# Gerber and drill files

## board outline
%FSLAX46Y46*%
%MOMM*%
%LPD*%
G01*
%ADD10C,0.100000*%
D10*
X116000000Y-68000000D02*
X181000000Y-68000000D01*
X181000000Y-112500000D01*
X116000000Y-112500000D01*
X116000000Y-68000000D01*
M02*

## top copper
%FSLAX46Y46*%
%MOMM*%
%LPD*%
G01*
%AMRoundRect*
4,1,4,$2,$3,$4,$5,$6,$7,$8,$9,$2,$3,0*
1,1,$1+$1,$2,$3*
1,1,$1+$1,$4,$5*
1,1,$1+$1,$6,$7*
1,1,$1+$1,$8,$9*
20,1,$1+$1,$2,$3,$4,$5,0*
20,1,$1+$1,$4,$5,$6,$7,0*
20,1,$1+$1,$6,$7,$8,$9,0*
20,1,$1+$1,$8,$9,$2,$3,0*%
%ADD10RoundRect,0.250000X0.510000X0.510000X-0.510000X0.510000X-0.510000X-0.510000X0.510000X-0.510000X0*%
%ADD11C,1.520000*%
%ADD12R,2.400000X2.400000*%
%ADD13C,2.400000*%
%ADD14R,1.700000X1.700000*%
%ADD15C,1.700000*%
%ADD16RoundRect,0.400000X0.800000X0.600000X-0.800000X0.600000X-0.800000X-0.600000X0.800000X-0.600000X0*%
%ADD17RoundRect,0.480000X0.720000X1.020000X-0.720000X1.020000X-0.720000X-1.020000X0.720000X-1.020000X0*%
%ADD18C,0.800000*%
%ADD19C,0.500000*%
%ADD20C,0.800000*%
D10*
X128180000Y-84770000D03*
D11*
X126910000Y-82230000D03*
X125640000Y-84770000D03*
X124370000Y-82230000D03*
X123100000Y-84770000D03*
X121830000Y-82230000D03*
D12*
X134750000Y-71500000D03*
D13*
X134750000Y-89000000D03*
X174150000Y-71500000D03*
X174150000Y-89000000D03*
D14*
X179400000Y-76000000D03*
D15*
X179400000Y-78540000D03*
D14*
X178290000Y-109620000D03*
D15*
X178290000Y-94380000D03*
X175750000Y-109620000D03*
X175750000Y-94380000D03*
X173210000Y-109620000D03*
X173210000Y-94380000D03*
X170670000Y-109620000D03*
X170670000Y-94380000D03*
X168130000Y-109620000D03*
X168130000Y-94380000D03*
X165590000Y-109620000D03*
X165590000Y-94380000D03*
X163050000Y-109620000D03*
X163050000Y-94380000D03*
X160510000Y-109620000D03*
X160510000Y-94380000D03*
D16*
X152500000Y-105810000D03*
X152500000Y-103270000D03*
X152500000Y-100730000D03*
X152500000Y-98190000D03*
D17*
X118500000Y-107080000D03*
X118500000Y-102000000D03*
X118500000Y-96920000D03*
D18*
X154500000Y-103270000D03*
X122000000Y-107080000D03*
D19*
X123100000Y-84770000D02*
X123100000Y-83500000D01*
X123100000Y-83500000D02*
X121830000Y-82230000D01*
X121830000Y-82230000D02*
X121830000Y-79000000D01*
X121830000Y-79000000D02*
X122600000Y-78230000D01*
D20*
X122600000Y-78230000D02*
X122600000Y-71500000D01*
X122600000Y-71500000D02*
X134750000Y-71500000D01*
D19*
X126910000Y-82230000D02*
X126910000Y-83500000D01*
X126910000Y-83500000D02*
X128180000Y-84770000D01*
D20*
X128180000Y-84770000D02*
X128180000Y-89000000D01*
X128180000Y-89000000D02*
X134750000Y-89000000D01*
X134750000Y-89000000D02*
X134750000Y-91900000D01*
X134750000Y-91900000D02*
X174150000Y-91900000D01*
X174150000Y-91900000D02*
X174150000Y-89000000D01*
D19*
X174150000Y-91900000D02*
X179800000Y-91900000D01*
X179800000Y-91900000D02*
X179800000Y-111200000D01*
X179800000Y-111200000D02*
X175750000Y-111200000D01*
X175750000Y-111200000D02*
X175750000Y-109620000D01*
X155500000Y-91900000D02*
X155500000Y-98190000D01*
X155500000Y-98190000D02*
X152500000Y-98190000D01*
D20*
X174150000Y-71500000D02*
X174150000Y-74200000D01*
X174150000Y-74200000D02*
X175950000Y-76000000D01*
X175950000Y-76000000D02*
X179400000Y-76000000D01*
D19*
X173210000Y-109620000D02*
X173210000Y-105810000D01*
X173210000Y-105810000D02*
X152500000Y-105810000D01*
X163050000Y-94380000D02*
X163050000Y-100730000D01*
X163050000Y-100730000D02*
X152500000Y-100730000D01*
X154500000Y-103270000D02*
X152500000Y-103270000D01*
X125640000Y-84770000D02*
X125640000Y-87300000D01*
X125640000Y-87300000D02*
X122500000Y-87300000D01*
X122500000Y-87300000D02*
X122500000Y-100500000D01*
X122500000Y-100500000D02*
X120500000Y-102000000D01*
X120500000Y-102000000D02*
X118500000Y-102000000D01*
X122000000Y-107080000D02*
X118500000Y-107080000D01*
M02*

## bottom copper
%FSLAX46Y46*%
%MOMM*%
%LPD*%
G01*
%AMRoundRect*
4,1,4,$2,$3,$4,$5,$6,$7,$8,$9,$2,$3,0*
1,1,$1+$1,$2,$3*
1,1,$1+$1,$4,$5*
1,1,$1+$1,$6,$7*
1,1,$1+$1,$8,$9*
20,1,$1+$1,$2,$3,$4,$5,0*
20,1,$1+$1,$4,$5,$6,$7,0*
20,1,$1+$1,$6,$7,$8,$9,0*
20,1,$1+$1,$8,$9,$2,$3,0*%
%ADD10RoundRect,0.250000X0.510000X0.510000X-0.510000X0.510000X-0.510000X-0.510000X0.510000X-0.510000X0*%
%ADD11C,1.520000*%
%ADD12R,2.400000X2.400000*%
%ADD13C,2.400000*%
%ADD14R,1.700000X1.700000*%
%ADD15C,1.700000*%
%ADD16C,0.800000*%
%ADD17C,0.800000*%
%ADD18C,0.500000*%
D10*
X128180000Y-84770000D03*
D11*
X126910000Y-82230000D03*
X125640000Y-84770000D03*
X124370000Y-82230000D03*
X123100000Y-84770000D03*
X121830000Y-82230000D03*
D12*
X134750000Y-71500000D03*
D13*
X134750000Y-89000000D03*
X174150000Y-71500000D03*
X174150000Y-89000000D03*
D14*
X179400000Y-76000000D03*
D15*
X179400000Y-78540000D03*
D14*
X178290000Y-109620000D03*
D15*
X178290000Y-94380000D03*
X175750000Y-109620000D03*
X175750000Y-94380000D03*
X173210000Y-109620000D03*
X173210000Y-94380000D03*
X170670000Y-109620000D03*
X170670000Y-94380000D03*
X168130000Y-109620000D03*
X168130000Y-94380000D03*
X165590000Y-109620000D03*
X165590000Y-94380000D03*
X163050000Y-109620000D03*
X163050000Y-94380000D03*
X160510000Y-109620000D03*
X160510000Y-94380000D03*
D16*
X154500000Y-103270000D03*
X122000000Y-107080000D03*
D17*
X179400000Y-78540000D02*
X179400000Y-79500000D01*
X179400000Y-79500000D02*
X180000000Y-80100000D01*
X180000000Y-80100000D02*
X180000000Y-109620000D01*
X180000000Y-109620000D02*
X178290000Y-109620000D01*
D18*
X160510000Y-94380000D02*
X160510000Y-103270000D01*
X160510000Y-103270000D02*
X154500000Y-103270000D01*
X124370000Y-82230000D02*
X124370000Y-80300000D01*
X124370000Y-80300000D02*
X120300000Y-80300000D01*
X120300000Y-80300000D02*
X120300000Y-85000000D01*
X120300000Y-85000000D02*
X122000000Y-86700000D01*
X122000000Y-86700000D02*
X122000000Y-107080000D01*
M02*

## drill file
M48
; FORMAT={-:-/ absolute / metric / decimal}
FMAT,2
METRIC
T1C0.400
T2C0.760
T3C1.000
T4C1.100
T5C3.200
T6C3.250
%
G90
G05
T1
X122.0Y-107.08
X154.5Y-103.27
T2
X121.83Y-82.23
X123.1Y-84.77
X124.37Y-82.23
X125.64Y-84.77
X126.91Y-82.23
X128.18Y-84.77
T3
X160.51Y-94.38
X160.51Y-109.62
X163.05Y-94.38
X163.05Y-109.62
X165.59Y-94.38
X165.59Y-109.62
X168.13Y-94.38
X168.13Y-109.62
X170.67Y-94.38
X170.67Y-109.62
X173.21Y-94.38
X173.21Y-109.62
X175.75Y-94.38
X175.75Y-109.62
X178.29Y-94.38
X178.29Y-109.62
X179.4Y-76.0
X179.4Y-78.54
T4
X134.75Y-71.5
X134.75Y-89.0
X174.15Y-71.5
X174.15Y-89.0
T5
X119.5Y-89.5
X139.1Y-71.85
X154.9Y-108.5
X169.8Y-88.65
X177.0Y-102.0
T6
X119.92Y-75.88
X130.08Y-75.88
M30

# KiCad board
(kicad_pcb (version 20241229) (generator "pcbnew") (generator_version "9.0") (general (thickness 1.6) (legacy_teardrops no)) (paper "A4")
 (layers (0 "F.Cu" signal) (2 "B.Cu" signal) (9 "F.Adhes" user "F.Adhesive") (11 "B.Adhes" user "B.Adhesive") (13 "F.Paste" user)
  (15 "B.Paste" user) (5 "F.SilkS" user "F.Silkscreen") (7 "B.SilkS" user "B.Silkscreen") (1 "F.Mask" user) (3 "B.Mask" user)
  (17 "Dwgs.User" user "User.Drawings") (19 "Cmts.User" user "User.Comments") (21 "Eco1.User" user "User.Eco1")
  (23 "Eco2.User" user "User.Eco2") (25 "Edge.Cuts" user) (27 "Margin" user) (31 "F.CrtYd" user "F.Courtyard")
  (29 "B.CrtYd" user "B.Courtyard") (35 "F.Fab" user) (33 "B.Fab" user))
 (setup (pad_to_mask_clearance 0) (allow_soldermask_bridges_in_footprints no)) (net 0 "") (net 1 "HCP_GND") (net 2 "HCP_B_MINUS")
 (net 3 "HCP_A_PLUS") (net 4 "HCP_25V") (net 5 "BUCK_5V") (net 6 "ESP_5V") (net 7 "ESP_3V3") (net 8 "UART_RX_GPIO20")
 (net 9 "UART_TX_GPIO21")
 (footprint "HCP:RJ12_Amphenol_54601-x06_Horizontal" (layer "F.Cu") (at 128.18 84.77 180)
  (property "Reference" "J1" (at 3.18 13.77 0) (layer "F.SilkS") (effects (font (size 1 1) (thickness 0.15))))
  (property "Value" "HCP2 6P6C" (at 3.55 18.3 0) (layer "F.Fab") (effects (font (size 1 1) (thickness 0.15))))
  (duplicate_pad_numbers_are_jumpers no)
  (pad "" np_thru_hole circle (at -1.9 8.89 180) (size 3.25 3.25) (drill 3.25) (layers "*.Cu" "*.Mask"))
  (pad "" np_thru_hole circle (at 8.26 8.89 180) (size 3.25 3.25) (drill 3.25) (layers "*.Cu" "*.Mask"))
  (pad "1" thru_hole roundrect (at 0 0 180) (size 1.52 1.52) (drill 0.76) (layers "*.Cu" "*.Mask") (remove_unused_layers no)
   (roundrect_rratio 0.1644736842) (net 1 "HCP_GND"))
  (pad "2" thru_hole circle (at 1.27 2.54 180) (size 1.52 1.52) (drill 0.76) (layers "*.Cu" "*.Mask") (remove_unused_layers no)
   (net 1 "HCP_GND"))
  (pad "3" thru_hole circle (at 2.54 0 180) (size 1.52 1.52) (drill 0.76) (layers "*.Cu" "*.Mask") (remove_unused_layers no)
   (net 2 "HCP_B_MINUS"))
  (pad "4" thru_hole circle (at 3.81 2.54 180) (size 1.52 1.52) (drill 0.76) (layers "*.Cu" "*.Mask") (remove_unused_layers no)
   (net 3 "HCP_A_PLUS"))
  (pad "5" thru_hole circle (at 5.08 0 180) (size 1.52 1.52) (drill 0.76) (layers "*.Cu" "*.Mask") (remove_unused_layers no)
   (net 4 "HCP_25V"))
  (pad "6" thru_hole circle (at 6.35 2.54 180) (size 1.52 1.52) (drill 0.76) (layers "*.Cu" "*.Mask") (remove_unused_layers no)
   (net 4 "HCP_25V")))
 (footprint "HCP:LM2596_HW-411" (layer "F.Cu") (at 154.45 80.25 0)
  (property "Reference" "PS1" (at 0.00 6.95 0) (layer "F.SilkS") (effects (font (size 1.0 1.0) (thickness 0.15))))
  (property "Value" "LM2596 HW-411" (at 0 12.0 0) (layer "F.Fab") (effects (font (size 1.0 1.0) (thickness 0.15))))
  (pad "1" thru_hole rect (at -19.7 -8.75) (size 2.4 2.4) (drill 1.1) (layers "*.Cu" "*.Mask") (remove_unused_layers no) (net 4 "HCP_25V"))
  (pad "2" thru_hole circle (at -19.7 8.75) (size 2.4 2.4) (drill 1.1) (layers "*.Cu" "*.Mask") (remove_unused_layers no) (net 1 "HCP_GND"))
  (pad "3" thru_hole circle (at 19.7 -8.75) (size 2.4 2.4) (drill 1.1) (layers "*.Cu" "*.Mask") (remove_unused_layers no) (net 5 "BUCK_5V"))
  (pad "4" thru_hole circle (at 19.7 8.75) (size 2.4 2.4) (drill 1.1) (layers "*.Cu" "*.Mask") (remove_unused_layers no) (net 1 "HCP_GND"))
  (pad "" np_thru_hole circle (at -15.35 -8.4) (size 3.2 3.2) (drill 3.2) (layers "*.Cu" "*.Mask"))
  (pad "" np_thru_hole circle (at 15.35 8.4) (size 3.2 3.2) (drill 3.2) (layers "*.Cu" "*.Mask")))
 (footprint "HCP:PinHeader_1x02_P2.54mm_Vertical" (layer "F.Cu") (at 179.4 76.0 0)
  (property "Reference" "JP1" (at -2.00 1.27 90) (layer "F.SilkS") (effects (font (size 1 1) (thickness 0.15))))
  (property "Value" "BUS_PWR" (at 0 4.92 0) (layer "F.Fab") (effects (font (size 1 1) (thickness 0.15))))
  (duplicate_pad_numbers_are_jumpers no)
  (pad "1" thru_hole rect (at 0 0) (size 1.7 1.7) (drill 1) (layers "*.Cu" "*.Mask") (remove_unused_layers no) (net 5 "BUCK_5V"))
  (pad "2" thru_hole circle (at 0 2.54) (size 1.7 1.7) (drill 1) (layers "*.Cu" "*.Mask") (remove_unused_layers no) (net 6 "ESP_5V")))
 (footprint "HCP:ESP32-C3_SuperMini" (layer "F.Cu") (at 169.4 102.0 270)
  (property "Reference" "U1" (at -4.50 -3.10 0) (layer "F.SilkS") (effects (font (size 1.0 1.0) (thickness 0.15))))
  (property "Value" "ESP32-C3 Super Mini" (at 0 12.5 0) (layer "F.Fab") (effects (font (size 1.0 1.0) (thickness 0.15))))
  (pad "1" thru_hole rect (at 7.62 -8.89 270) (size 1.7 1.7) (drill 1.0) (layers "*.Cu" "*.Mask") (remove_unused_layers no) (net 6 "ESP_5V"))
  (pad "2" thru_hole circle (at -7.62 -8.89 270) (size 1.7 1.7) (drill 1.0) (layers "*.Cu" "*.Mask") (remove_unused_layers no))
  (pad "3" thru_hole circle (at 7.62 -6.35 270) (size 1.7 1.7) (drill 1.0) (layers "*.Cu" "*.Mask") (remove_unused_layers no)
   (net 1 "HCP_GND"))
  (pad "4" thru_hole circle (at -7.62 -6.35 270) (size 1.7 1.7) (drill 1.0) (layers "*.Cu" "*.Mask") (remove_unused_layers no))
  (pad "5" thru_hole circle (at 7.62 -3.81 270) (size 1.7 1.7) (drill 1.0) (layers "*.Cu" "*.Mask") (remove_unused_layers no)
   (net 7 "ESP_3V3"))
  (pad "6" thru_hole circle (at -7.62 -3.81 270) (size 1.7 1.7) (drill 1.0) (layers "*.Cu" "*.Mask") (remove_unused_layers no))
  (pad "7" thru_hole circle (at 7.62 -1.27 270) (size 1.7 1.7) (drill 1.0) (layers "*.Cu" "*.Mask") (remove_unused_layers no))
  (pad "8" thru_hole circle (at -7.62 -1.27 270) (size 1.7 1.7) (drill 1.0) (layers "*.Cu" "*.Mask") (remove_unused_layers no))
  (pad "9" thru_hole circle (at 7.62 1.27 270) (size 1.7 1.7) (drill 1.0) (layers "*.Cu" "*.Mask") (remove_unused_layers no))
  (pad "10" thru_hole circle (at -7.62 1.27 270) (size 1.7 1.7) (drill 1.0) (layers "*.Cu" "*.Mask") (remove_unused_layers no))
  (pad "11" thru_hole circle (at 7.62 3.81 270) (size 1.7 1.7) (drill 1.0) (layers "*.Cu" "*.Mask") (remove_unused_layers no))
  (pad "12" thru_hole circle (at -7.62 3.81 270) (size 1.7 1.7) (drill 1.0) (layers "*.Cu" "*.Mask") (remove_unused_layers no))
  (pad "13" thru_hole circle (at 7.62 6.35 270) (size 1.7 1.7) (drill 1.0) (layers "*.Cu" "*.Mask") (remove_unused_layers no))
  (pad "14" thru_hole circle (at -7.62 6.35 270) (size 1.7 1.7) (drill 1.0) (layers "*.Cu" "*.Mask") (remove_unused_layers no)
   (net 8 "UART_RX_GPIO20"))
  (pad "15" thru_hole circle (at 7.62 8.89 270) (size 1.7 1.7) (drill 1.0) (layers "*.Cu" "*.Mask") (remove_unused_layers no))
  (pad "16" thru_hole circle (at -7.62 8.89 270) (size 1.7 1.7) (drill 1.0) (layers "*.Cu" "*.Mask") (remove_unused_layers no)
   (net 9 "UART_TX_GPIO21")))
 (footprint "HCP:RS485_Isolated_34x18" (layer "F.Cu") (at 135.5 102.0 180)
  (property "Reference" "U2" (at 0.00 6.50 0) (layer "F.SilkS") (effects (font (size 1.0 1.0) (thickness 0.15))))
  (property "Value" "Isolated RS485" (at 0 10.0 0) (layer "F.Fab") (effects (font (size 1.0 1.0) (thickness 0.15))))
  (pad "1" smd roundrect (at -17 -3.81 180) (size 2.4 2.0) (layers "F.Cu" "F.Paste" "F.Mask") (roundrect_rratio 0.2) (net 7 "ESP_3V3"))
  (pad "2" smd roundrect (at -17 -1.27 180) (size 2.4 2.0) (layers "F.Cu" "F.Paste" "F.Mask") (roundrect_rratio 0.2)
   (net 9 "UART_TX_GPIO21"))
  (pad "3" smd roundrect (at -17 1.27 180) (size 2.4 2.0) (layers "F.Cu" "F.Paste" "F.Mask") (roundrect_rratio 0.2) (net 8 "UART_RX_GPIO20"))
  (pad "4" smd roundrect (at -17 3.81 180) (size 2.4 2.0) (layers "F.Cu" "F.Paste" "F.Mask") (roundrect_rratio 0.2) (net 1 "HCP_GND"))
  (pad "5" smd roundrect (at 17 -5.08 180) (size 2.4 3.0) (layers "F.Cu" "F.Paste" "F.Mask") (roundrect_rratio 0.2) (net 3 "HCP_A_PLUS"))
  (pad "6" smd roundrect (at 17 0 180) (size 2.4 3.0) (layers "F.Cu" "F.Paste" "F.Mask") (roundrect_rratio 0.2) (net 2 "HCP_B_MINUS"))
  (pad "7" smd roundrect (at 17 5.08 180) (size 2.4 3.0) (layers "F.Cu" "F.Paste" "F.Mask") (roundrect_rratio 0.2)))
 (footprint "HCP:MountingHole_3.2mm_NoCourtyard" (layer "F.Cu") (at 119.5 89.5 0)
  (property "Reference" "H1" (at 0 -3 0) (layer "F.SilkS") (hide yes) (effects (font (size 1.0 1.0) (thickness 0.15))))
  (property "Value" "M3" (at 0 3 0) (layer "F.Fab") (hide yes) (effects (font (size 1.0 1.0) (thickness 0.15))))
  (pad "" np_thru_hole circle (at 0 0) (size 3.2 3.2) (drill 3.2) (layers "*.Cu" "*.Mask")))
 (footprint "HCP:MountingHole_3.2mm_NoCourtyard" (layer "F.Cu") (at 154.9 108.5 0)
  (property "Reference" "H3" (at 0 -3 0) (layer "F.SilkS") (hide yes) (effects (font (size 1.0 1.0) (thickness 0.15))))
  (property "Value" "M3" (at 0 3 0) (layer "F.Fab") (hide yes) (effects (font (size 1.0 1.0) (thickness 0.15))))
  (pad "" np_thru_hole circle (at 0 0) (size 3.2 3.2) (drill 3.2) (layers "*.Cu" "*.Mask")))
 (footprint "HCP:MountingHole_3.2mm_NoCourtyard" (layer "F.Cu") (at 177.0 102.0 0)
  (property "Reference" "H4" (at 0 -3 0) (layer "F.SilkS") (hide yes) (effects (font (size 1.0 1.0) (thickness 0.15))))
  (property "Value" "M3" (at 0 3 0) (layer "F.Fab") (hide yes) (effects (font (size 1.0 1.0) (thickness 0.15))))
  (pad "" np_thru_hole circle (at 0 0) (size 3.2 3.2) (drill 3.2) (layers "*.Cu" "*.Mask")))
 (segment (start 123.1 84.77) (end 123.1 83.5) (width 0.5) (layer "F.Cu") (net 4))
 (segment (start 123.1 83.5) (end 121.83 82.23) (width 0.5) (layer "F.Cu") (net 4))
 (segment (start 121.83 82.23) (end 121.83 79.0) (width 0.5) (layer "F.Cu") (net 4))
 (segment (start 121.83 79.0) (end 122.6 78.23) (width 0.5) (layer "F.Cu") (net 4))
 (segment (start 122.6 78.23) (end 122.6 71.5) (width 0.8) (layer "F.Cu") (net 4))
 (segment (start 122.6 71.5) (end 134.75 71.5) (width 0.8) (layer "F.Cu") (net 4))
 (segment (start 126.91 82.23) (end 126.91 83.5) (width 0.5) (layer "F.Cu") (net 1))
 (segment (start 126.91 83.5) (end 128.18 84.77) (width 0.5) (layer "F.Cu") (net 1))
 (segment (start 128.18 84.77) (end 128.18 89.0) (width 0.8) (layer "F.Cu") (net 1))
 (segment (start 128.18 89.0) (end 134.75 89.0) (width 0.8) (layer "F.Cu") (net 1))
 (segment (start 134.75 89.0) (end 134.75 91.9) (width 0.8) (layer "F.Cu") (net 1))
 (segment (start 134.75 91.9) (end 174.15 91.9) (width 0.8) (layer "F.Cu") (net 1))
 (segment (start 174.15 91.9) (end 174.15 89.0) (width 0.8) (layer "F.Cu") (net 1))
 (segment (start 174.15 91.9) (end 179.8 91.9) (width 0.5) (layer "F.Cu") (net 1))
 (segment (start 179.8 91.9) (end 179.8 111.2) (width 0.5) (layer "F.Cu") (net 1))
 (segment (start 179.8 111.2) (end 175.75 111.2) (width 0.5) (layer "F.Cu") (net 1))
 (segment (start 175.75 111.2) (end 175.75 109.62) (width 0.5) (layer "F.Cu") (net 1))
 (segment (start 155.5 91.9) (end 155.5 98.19) (width 0.5) (layer "F.Cu") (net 1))
 (segment (start 155.5 98.19) (end 152.5 98.19) (width 0.5) (layer "F.Cu") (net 1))
 (segment (start 174.15 71.5) (end 174.15 74.2) (width 0.8) (layer "F.Cu") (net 5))
 (segment (start 174.15 74.2) (end 175.95 76.0) (width 0.8) (layer "F.Cu") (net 5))
 (segment (start 175.95 76.0) (end 179.4 76.0) (width 0.8) (layer "F.Cu") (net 5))
 (segment (start 179.4 78.54) (end 179.4 79.5) (width 0.8) (layer "B.Cu") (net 6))
 (segment (start 179.4 79.5) (end 180.0 80.1) (width 0.8) (layer "B.Cu") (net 6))
 (segment (start 180.0 80.1) (end 180.0 109.62) (width 0.8) (layer "B.Cu") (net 6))
 (segment (start 180.0 109.62) (end 178.29 109.62) (width 0.8) (layer "B.Cu") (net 6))
 (segment (start 173.21 109.62) (end 173.21 105.81) (width 0.5) (layer "F.Cu") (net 7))
 (segment (start 173.21 105.81) (end 152.5 105.81) (width 0.5) (layer "F.Cu") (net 7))
 (segment (start 163.05 94.38) (end 163.05 100.73) (width 0.5) (layer "F.Cu") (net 8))
 (segment (start 163.05 100.73) (end 152.5 100.73) (width 0.5) (layer "F.Cu") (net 8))
 (segment (start 160.51 94.38) (end 160.51 103.27) (width 0.5) (layer "B.Cu") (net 9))
 (segment (start 160.51 103.27) (end 154.5 103.27) (width 0.5) (layer "B.Cu") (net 9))
 (segment (start 154.5 103.27) (end 152.5 103.27) (width 0.5) (layer "F.Cu") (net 9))
 (segment (start 125.64 84.77) (end 125.64 87.3) (width 0.5) (layer "F.Cu") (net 2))
 (segment (start 125.64 87.3) (end 122.5 87.3) (width 0.5) (layer "F.Cu") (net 2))
 (segment (start 122.5 87.3) (end 122.5 100.5) (width 0.5) (layer "F.Cu") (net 2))
 (segment (start 122.5 100.5) (end 120.5 102.0) (width 0.5) (layer "F.Cu") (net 2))
 (segment (start 120.5 102.0) (end 118.5 102.0) (width 0.5) (layer "F.Cu") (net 2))
 (segment (start 124.37 82.23) (end 124.37 80.3) (width 0.5) (layer "B.Cu") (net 3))
 (segment (start 124.37 80.3) (end 120.3 80.3) (width 0.5) (layer "B.Cu") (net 3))
 (segment (start 120.3 80.3) (end 120.3 85.0) (width 0.5) (layer "B.Cu") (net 3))
 (segment (start 120.3 85.0) (end 122.0 86.7) (width 0.5) (layer "B.Cu") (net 3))
 (segment (start 122.0 86.7) (end 122.0 107.08) (width 0.5) (layer "B.Cu") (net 3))
 (segment (start 122.0 107.08) (end 118.5 107.08) (width 0.5) (layer "F.Cu") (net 3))
 (via (at 154.5 103.27) (size 0.8) (drill 0.4) (layers "F.Cu" "B.Cu") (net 9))
 (via (at 122.0 107.08) (size 0.8) (drill 0.4) (layers "F.Cu" "B.Cu") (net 3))
 (gr_rect (start 116.0 68.0) (end 181.0 112.5) (stroke (width 0.1) (type default)) (fill none) (layer "Edge.Cuts")))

